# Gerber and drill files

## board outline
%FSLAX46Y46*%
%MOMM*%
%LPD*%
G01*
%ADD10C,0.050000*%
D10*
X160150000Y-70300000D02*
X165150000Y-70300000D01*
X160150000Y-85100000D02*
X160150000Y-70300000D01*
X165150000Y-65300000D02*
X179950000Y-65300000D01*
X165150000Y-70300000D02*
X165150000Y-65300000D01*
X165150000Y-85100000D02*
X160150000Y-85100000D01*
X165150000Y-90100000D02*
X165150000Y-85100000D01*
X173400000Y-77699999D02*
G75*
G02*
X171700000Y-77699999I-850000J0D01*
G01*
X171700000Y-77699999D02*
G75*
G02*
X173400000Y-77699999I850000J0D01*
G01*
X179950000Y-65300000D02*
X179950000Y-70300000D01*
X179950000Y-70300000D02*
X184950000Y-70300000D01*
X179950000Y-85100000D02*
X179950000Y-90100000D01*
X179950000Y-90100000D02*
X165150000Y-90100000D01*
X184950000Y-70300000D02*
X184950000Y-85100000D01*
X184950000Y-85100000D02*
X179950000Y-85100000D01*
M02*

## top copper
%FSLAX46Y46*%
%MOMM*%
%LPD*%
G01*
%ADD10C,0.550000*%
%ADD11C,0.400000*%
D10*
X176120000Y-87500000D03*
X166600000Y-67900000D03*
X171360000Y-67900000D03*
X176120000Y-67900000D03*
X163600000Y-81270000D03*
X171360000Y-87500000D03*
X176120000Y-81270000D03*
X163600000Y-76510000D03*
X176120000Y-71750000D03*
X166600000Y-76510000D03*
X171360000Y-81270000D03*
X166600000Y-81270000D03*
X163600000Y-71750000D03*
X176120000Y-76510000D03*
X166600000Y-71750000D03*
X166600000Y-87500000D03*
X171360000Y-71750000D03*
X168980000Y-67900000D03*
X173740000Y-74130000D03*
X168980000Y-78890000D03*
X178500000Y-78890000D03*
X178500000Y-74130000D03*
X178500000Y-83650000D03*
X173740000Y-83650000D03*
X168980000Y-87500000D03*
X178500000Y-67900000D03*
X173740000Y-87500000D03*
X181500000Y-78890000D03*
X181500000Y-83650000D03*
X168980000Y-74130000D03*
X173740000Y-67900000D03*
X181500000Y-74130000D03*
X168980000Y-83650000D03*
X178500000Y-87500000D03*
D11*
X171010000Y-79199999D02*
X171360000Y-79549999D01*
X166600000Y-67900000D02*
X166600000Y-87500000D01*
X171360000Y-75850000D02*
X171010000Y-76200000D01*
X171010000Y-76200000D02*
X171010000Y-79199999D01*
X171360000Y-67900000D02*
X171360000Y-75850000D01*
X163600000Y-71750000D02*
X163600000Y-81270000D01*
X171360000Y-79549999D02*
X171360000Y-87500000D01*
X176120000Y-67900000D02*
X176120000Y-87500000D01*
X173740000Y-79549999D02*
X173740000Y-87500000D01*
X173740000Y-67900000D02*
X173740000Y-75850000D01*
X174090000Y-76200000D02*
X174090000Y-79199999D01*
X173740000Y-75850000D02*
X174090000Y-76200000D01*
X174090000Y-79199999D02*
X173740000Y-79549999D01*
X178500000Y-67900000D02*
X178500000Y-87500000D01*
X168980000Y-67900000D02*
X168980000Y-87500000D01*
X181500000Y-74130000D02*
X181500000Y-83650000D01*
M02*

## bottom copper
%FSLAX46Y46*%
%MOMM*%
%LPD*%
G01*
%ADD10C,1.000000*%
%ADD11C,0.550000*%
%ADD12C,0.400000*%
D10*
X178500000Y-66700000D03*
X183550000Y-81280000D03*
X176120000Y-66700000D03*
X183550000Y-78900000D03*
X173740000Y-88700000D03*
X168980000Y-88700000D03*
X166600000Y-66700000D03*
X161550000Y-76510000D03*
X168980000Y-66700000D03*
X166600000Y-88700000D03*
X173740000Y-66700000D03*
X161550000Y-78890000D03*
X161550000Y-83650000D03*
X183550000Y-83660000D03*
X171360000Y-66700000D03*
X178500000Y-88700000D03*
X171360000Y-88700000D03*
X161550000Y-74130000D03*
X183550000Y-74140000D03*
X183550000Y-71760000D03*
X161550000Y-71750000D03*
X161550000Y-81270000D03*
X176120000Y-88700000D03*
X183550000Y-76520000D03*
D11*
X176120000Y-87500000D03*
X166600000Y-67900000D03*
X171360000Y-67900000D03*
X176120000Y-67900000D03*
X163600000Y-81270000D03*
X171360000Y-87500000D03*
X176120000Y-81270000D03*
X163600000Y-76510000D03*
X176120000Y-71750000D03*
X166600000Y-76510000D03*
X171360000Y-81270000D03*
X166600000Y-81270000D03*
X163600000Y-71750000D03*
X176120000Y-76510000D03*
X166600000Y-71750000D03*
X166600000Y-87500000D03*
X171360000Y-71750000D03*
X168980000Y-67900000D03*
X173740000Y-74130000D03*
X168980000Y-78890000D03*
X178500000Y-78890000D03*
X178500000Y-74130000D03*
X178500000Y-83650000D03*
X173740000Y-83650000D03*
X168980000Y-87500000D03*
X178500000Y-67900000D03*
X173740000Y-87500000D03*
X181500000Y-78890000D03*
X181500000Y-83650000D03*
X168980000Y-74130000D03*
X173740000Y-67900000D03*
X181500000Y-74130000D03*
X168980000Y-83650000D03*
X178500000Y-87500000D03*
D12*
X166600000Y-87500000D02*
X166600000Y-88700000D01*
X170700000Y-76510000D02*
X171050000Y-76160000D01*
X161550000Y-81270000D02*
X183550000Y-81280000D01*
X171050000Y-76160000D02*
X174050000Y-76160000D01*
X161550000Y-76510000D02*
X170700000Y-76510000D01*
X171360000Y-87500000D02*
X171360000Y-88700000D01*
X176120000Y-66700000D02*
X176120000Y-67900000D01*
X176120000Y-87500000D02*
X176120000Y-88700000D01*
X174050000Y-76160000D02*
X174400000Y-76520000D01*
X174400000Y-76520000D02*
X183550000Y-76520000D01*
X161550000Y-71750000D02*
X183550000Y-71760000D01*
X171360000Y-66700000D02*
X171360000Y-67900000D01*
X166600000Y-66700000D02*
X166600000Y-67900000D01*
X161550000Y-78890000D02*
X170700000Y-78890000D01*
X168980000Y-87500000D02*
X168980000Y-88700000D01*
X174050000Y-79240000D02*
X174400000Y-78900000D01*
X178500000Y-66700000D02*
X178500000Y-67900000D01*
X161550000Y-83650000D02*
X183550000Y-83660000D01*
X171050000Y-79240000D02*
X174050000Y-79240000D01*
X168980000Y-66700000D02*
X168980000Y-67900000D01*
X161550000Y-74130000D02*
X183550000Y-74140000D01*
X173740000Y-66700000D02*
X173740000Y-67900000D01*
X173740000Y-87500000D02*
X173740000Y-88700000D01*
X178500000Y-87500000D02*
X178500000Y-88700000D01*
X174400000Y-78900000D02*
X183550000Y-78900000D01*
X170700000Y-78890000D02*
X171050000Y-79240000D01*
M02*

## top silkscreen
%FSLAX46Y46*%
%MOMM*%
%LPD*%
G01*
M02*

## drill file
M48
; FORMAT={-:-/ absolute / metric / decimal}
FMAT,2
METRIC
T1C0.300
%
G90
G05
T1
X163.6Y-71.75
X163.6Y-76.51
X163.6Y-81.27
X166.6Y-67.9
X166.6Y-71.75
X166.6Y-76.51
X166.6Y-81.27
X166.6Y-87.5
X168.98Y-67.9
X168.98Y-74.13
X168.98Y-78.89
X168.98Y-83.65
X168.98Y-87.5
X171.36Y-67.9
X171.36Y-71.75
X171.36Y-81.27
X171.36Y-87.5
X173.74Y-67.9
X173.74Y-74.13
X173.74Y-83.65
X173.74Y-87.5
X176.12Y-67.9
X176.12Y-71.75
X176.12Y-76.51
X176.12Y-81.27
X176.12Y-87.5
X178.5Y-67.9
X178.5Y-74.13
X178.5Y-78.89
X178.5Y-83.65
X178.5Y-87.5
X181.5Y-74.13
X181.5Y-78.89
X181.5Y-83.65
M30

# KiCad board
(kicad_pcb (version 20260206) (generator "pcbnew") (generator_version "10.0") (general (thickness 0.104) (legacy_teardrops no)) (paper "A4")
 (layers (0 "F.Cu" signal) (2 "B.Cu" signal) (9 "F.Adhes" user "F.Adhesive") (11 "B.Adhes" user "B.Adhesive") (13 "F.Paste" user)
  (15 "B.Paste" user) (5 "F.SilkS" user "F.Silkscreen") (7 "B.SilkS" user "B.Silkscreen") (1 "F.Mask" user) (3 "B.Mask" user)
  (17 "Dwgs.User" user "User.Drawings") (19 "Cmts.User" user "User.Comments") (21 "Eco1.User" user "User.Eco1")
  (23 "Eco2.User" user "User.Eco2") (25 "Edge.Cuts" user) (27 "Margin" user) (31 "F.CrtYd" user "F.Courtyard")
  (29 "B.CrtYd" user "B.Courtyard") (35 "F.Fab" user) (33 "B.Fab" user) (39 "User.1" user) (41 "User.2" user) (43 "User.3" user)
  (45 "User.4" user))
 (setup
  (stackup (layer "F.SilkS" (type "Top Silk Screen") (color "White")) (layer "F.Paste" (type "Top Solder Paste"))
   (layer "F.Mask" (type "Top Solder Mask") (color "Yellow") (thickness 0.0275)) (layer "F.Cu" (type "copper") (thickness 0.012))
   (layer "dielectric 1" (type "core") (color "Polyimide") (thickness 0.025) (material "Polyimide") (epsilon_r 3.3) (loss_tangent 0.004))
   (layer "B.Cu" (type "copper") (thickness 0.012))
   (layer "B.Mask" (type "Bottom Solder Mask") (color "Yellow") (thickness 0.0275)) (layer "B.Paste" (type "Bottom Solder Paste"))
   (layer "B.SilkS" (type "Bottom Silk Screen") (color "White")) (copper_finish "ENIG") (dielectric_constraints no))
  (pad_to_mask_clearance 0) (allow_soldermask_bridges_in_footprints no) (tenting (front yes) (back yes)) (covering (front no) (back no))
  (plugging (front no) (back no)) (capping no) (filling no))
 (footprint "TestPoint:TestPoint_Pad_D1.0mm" (layer "B.Cu") (at 178.5 66.7 180)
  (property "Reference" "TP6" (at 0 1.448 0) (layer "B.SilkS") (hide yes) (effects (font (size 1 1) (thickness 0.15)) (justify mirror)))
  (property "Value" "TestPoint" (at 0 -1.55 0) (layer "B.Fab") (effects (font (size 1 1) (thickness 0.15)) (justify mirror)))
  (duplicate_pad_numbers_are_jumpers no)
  (pad "1" smd circle (at 0 0 180) (size 1 1) (layers "B.Cu" "B.Mask") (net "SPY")))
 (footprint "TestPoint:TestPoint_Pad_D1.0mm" (layer "B.Cu") (at 183.55 81.28 90)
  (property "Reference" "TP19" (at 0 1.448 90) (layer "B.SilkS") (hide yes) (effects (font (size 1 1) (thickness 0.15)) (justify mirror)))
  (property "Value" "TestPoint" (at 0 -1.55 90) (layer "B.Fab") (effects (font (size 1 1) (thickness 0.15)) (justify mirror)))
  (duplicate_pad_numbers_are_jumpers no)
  (pad "1" smd circle (at 0 0 90) (size 1 1) (layers "B.Cu" "B.Mask") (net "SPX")))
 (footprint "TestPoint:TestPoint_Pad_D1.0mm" (layer "B.Cu") (at 176.12 66.7 180)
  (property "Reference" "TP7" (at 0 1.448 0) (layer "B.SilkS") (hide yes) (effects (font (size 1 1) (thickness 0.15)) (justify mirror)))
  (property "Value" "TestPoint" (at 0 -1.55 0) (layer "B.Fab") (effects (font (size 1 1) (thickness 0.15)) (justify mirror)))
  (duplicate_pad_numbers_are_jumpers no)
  (pad "1" smd circle (at 0 0 180) (size 1 1) (layers "B.Cu" "B.Mask") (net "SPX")))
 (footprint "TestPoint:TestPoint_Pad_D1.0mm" (layer "B.Cu") (at 183.55 78.9 90)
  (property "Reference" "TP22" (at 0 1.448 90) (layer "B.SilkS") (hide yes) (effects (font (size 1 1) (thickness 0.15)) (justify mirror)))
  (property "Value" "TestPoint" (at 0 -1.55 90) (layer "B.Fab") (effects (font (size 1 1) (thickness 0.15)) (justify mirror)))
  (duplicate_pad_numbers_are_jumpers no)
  (pad "1" smd circle (at 0 0 90) (size 1 1) (layers "B.Cu" "B.Mask") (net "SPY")))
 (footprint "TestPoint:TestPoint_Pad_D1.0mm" (layer "B.Cu") (at 173.74 88.7)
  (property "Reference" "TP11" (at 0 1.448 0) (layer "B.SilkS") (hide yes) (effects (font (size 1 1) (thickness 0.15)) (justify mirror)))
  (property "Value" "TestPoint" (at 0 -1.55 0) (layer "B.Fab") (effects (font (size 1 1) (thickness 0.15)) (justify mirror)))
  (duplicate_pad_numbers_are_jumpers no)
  (pad "1" smd circle (at 0 0) (size 1 1) (layers "B.Cu" "B.Mask") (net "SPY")))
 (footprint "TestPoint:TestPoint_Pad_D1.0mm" (layer "B.Cu") (at 168.98 88.7)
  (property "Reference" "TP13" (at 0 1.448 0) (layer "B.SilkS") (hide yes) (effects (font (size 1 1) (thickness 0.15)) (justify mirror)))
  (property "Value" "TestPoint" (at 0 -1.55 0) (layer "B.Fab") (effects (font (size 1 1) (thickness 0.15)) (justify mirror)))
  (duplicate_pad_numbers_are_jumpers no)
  (pad "1" smd circle (at 0 0) (size 1 1) (layers "B.Cu" "B.Mask") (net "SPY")))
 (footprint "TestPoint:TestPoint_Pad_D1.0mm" (layer "B.Cu") (at 166.6 66.7 180)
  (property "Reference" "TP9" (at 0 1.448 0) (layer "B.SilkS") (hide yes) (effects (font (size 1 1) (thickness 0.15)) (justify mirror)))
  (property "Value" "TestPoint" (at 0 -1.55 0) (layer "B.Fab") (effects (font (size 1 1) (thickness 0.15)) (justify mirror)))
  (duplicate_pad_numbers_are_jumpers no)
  (pad "1" smd circle (at 0 0 180) (size 1 1) (layers "B.Cu" "B.Mask") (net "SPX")))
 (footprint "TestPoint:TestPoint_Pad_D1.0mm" (layer "B.Cu") (at 161.55 76.51 -90)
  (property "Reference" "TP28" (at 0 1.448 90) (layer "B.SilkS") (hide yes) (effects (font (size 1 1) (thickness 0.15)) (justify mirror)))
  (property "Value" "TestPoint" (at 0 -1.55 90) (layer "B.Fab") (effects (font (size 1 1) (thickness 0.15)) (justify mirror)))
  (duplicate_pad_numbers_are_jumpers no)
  (pad "1" smd circle (at 0 0 270) (size 1 1) (layers "B.Cu" "B.Mask") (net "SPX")))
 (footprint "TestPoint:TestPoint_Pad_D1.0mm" (layer "B.Cu") (at 168.98 66.7 180)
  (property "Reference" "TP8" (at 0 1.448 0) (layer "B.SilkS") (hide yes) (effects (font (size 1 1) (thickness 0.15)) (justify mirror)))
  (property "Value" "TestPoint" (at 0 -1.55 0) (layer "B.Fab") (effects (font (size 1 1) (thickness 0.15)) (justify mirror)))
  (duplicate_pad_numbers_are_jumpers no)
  (pad "1" smd circle (at 0 0 180) (size 1 1) (layers "B.Cu" "B.Mask") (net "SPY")))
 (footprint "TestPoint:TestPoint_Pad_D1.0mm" (layer "B.Cu") (at 166.6 88.7)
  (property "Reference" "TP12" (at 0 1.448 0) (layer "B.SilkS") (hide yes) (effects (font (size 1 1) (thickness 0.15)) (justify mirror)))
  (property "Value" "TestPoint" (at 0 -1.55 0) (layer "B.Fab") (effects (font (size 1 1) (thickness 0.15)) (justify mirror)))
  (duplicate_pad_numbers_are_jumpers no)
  (pad "1" smd circle (at 0 0) (size 1 1) (layers "B.Cu" "B.Mask") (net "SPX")))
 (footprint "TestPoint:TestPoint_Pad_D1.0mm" (layer "B.Cu") (at 173.74 66.7 180)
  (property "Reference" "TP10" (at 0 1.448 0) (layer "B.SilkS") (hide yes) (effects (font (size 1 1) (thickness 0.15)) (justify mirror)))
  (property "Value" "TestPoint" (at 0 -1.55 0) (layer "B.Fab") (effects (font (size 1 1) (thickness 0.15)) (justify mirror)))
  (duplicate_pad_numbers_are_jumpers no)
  (pad "1" smd circle (at 0 0 180) (size 1 1) (layers "B.Cu" "B.Mask") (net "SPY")))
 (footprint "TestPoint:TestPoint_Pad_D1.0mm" (layer "B.Cu") (at 161.55 78.89 -90)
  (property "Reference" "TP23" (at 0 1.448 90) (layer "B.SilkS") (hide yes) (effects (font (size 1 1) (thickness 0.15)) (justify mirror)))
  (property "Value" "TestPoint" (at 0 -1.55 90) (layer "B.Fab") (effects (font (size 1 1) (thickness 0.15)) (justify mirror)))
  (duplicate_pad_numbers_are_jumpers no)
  (pad "1" smd circle (at 0 0 270) (size 1 1) (layers "B.Cu" "B.Mask") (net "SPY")))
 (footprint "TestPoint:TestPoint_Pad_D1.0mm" (layer "B.Cu") (at 161.55 83.65 -90)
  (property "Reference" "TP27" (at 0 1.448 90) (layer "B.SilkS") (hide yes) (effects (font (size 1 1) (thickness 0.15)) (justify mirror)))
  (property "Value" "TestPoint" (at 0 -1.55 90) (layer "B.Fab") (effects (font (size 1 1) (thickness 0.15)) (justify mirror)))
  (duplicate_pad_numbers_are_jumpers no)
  (pad "1" smd circle (at 0 0 270) (size 1 1) (layers "B.Cu" "B.Mask") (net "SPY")))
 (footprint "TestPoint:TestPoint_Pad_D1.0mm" (layer "B.Cu") (at 183.55 83.66 90)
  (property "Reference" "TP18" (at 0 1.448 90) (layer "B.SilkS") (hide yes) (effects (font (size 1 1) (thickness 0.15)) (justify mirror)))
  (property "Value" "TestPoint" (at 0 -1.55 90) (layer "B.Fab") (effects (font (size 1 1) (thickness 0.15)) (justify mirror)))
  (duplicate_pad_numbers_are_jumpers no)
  (pad "1" smd circle (at 0 0 90) (size 1 1) (layers "B.Cu" "B.Mask") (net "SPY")))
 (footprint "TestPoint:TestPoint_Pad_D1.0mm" (layer "B.Cu") (at 171.36 66.7 180)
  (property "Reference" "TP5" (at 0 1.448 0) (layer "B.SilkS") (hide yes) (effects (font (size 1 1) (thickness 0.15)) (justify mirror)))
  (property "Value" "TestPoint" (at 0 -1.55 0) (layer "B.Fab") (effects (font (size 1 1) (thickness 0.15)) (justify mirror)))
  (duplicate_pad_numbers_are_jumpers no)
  (pad "1" smd circle (at 0 0 180) (size 1 1) (layers "B.Cu" "B.Mask") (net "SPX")))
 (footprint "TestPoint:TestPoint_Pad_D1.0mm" (layer "B.Cu") (at 178.5 88.7)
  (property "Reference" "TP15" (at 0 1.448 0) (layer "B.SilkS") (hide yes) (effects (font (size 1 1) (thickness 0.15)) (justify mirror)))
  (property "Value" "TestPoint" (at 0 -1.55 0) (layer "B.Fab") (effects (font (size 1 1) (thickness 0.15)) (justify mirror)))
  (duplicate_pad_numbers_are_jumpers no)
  (pad "1" smd circle (at 0 0) (size 1 1) (layers "B.Cu" "B.Mask") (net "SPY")))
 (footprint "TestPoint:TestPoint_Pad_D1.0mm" (layer "B.Cu") (at 171.36 88.7)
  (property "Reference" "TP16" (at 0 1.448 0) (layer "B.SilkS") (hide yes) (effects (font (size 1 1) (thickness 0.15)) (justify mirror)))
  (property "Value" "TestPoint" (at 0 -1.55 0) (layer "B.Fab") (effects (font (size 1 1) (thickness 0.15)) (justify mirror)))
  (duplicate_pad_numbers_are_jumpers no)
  (pad "1" smd circle (at 0 0) (size 1 1) (layers "B.Cu" "B.Mask") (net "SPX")))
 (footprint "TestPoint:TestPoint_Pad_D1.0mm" (layer "B.Cu") (at 161.55 74.13 -90)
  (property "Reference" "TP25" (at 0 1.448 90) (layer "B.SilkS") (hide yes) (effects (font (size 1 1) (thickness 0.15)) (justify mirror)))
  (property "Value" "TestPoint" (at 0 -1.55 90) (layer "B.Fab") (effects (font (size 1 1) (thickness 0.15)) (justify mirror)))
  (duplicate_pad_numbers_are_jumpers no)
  (pad "1" smd circle (at 0 0 270) (size 1 1) (layers "B.Cu" "B.Mask") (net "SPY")))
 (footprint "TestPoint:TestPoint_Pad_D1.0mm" (layer "B.Cu") (at 183.55 74.14 90)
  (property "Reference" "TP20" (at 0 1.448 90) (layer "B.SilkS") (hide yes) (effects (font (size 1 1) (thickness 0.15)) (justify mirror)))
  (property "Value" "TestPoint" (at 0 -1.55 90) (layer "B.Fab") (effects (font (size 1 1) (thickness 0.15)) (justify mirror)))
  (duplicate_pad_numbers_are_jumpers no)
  (pad "1" smd circle (at 0 0 90) (size 1 1) (layers "B.Cu" "B.Mask") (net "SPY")))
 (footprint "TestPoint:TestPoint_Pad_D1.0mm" (layer "B.Cu") (at 183.55 71.76 90)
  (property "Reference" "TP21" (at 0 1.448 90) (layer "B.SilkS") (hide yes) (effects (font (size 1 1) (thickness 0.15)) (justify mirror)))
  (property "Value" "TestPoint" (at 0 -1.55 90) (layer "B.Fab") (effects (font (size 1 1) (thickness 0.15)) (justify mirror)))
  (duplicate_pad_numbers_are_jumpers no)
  (pad "1" smd circle (at 0 0 90) (size 1 1) (layers "B.Cu" "B.Mask") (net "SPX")))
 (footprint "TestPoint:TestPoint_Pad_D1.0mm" (layer "B.Cu") (at 161.55 71.75 -90)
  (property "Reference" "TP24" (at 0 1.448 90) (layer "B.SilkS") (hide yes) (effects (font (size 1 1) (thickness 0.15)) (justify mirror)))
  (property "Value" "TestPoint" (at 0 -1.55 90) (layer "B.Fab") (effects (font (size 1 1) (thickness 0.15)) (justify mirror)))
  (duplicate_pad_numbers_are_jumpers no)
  (pad "1" smd circle (at 0 0 270) (size 1 1) (layers "B.Cu" "B.Mask") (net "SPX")))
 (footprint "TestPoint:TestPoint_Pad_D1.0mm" (layer "B.Cu") (at 161.55 81.27 -90)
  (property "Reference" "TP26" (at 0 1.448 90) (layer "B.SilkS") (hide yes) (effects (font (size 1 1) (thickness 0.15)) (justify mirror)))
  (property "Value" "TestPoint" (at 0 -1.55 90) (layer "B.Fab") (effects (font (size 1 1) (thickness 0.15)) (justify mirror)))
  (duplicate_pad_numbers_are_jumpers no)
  (pad "1" smd circle (at 0 0 270) (size 1 1) (layers "B.Cu" "B.Mask") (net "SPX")))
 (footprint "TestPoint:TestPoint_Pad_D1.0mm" (layer "B.Cu") (at 176.12 88.7)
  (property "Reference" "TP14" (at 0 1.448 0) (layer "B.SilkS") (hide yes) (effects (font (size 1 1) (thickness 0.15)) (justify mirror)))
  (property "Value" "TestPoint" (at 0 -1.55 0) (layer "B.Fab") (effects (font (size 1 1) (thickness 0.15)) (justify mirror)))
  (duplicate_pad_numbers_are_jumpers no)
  (pad "1" smd circle (at 0 0) (size 1 1) (layers "B.Cu" "B.Mask") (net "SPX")))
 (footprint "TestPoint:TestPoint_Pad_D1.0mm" (layer "B.Cu") (at 183.55 76.52 90)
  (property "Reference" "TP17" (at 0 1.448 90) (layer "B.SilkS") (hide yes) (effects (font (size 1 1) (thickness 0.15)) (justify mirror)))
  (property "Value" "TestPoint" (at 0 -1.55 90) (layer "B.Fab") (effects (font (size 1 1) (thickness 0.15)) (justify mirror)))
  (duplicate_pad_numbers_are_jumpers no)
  (pad "1" smd circle (at 0 0 90) (size 1 1) (layers "B.Cu" "B.Mask") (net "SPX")))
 (gr_line (start 160.15 70.3) (end 165.15 70.3) (stroke (width 0.05) (type default)) (layer "Edge.Cuts"))
 (gr_line (start 160.15 85.1) (end 160.15 70.3) (stroke (width 0.05) (type default)) (layer "Edge.Cuts"))
 (gr_line (start 165.15 65.3) (end 179.95 65.3) (stroke (width 0.05) (type default)) (layer "Edge.Cuts"))
 (gr_line (start 165.15 70.3) (end 165.15 65.3) (stroke (width 0.05) (type default)) (layer "Edge.Cuts"))
 (gr_line (start 165.15 85.1) (end 160.15 85.1) (stroke (width 0.05) (type default)) (layer "Edge.Cuts"))
 (gr_line (start 165.15 90.1) (end 165.15 85.1) (stroke (width 0.05) (type default)) (layer "Edge.Cuts"))
 (gr_circle (center 172.55 77.699999) (end 173.4 77.699999) (stroke (width 0.05) (type default)) (fill no) (layer "Edge.Cuts"))
 (gr_line (start 179.95 65.3) (end 179.95 70.3) (stroke (width 0.05) (type default)) (layer "Edge.Cuts"))
 (gr_line (start 179.95 70.3) (end 184.95 70.3) (stroke (width 0.05) (type default)) (layer "Edge.Cuts"))
 (gr_line (start 179.95 85.1) (end 179.95 90.1) (stroke (width 0.05) (type default)) (layer "Edge.Cuts"))
 (gr_line (start 179.95 90.1) (end 165.15 90.1) (stroke (width 0.05) (type default)) (layer "Edge.Cuts"))
 (gr_line (start 184.95 70.3) (end 184.95 85.1) (stroke (width 0.05) (type default)) (layer "Edge.Cuts"))
 (gr_line (start 184.95 85.1) (end 179.95 85.1) (stroke (width 0.05) (type default)) (layer "Edge.Cuts"))
 (segment (start 171.01 79.199999) (end 171.36 79.549999) (width 0.4) (layer "F.Cu") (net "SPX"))
 (segment (start 166.6 67.9) (end 166.6 87.5) (width 0.4) (layer "F.Cu") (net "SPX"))
 (segment (start 171.36 75.85) (end 171.01 76.2) (width 0.4) (layer "F.Cu") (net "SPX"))
 (segment (start 171.01 76.2) (end 171.01 79.199999) (width 0.4) (layer "F.Cu") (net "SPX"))
 (segment (start 171.36 67.9) (end 171.36 75.85) (width 0.4) (layer "F.Cu") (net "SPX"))
 (segment (start 163.6 71.75) (end 163.6 81.27) (width 0.4) (layer "F.Cu") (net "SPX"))
 (segment (start 171.36 79.549999) (end 171.36 87.5) (width 0.4) (layer "F.Cu") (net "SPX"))
 (segment (start 176.12 67.9) (end 176.12 87.5) (width 0.4) (layer "F.Cu") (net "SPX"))
 (via (at 176.12 87.5) (size 0.55) (drill 0.3) (layers "F.Cu" "B.Cu") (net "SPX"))
 (via (at 166.6 67.9) (size 0.55) (drill 0.3) (layers "F.Cu" "B.Cu") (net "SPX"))
 (via (at 171.36 67.9) (size 0.55) (drill 0.3) (layers "F.Cu" "B.Cu") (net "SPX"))
 (via (at 176.12 67.9) (size 0.55) (drill 0.3) (layers "F.Cu" "B.Cu") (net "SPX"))
 (via (at 163.6 81.27) (size 0.55) (drill 0.3) (layers "F.Cu" "B.Cu") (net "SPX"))
 (via (at 171.36 87.5) (size 0.55) (drill 0.3) (layers "F.Cu" "B.Cu") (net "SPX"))
 (via (at 176.12 81.27) (size 0.55) (drill 0.3) (layers "F.Cu" "B.Cu") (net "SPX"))
 (via (at 163.6 76.51) (size 0.55) (drill 0.3) (layers "F.Cu" "B.Cu") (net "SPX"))
 (via (at 176.12 71.75) (size 0.55) (drill 0.3) (layers "F.Cu" "B.Cu") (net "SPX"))
 (via (at 166.6 76.51) (size 0.55) (drill 0.3) (layers "F.Cu" "B.Cu") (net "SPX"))
 (via (at 171.36 81.27) (size 0.55) (drill 0.3) (layers "F.Cu" "B.Cu") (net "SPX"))
 (via (at 166.6 81.27) (size 0.55) (drill 0.3) (layers "F.Cu" "B.Cu") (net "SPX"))
 (via (at 163.6 71.75) (size 0.55) (drill 0.3) (layers "F.Cu" "B.Cu") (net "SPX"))
 (via (at 176.12 76.51) (size 0.55) (drill 0.3) (layers "F.Cu" "B.Cu") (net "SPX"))
 (via (at 166.6 71.75) (size 0.55) (drill 0.3) (layers "F.Cu" "B.Cu") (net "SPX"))
 (via (at 166.6 87.5) (size 0.55) (drill 0.3) (layers "F.Cu" "B.Cu") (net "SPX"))
 (via (at 171.36 71.75) (size 0.55) (drill 0.3) (layers "F.Cu" "B.Cu") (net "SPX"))
 (segment (start 166.6 87.5) (end 166.6 88.7) (width 0.4) (layer "B.Cu") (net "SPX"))
 (segment (start 170.7 76.51) (end 171.05 76.16) (width 0.4) (layer "B.Cu") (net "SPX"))
 (segment (start 161.55 81.27) (end 183.55 81.28) (width 0.4) (layer "B.Cu") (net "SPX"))
 (segment (start 171.05 76.16) (end 174.05 76.16) (width 0.4) (layer "B.Cu") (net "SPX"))
 (segment (start 161.55 76.51) (end 170.7 76.51) (width 0.4) (layer "B.Cu") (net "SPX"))
 (segment (start 171.36 87.5) (end 171.36 88.7) (width 0.4) (layer "B.Cu") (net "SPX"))
 (segment (start 176.12 66.7) (end 176.12 67.9) (width 0.4) (layer "B.Cu") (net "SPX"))
 (segment (start 176.12 87.5) (end 176.12 88.7) (width 0.4) (layer "B.Cu") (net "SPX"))
 (segment (start 174.05 76.16) (end 174.4 76.52) (width 0.4) (layer "B.Cu") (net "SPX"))
 (segment (start 174.4 76.52) (end 183.55 76.52) (width 0.4) (layer "B.Cu") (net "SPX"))
 (segment (start 161.55 71.75) (end 183.55 71.76) (width 0.4) (layer "B.Cu") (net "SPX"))
 (segment (start 171.36 66.7) (end 171.36 67.9) (width 0.4) (layer "B.Cu") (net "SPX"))
 (segment (start 166.6 66.7) (end 166.6 67.9) (width 0.4) (layer "B.Cu") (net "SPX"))
 (segment (start 173.74 79.549999) (end 173.74 87.5) (width 0.4) (layer "F.Cu") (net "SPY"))
 (segment (start 173.74 67.9) (end 173.74 75.85) (width 0.4) (layer "F.Cu") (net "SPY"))
 (segment (start 174.09 76.2) (end 174.09 79.199999) (width 0.4) (layer "F.Cu") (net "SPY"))
 (segment (start 173.74 75.85) (end 174.09 76.2) (width 0.4) (layer "F.Cu") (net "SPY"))
 (segment (start 174.09 79.199999) (end 173.74 79.549999) (width 0.4) (layer "F.Cu") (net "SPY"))
 (segment (start 178.5 67.9) (end 178.5 87.5) (width 0.4) (layer "F.Cu") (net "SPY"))
 (segment (start 168.98 67.9) (end 168.98 87.5) (width 0.4) (layer "F.Cu") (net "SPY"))
 (segment (start 181.5 74.13) (end 181.5 83.65) (width 0.4) (layer "F.Cu") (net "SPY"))
 (via (at 168.98 67.9) (size 0.55) (drill 0.3) (layers "F.Cu" "B.Cu") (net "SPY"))
 (via (at 173.74 74.13) (size 0.55) (drill 0.3) (layers "F.Cu" "B.Cu") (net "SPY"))
 (via (at 168.98 78.89) (size 0.55) (drill 0.3) (layers "F.Cu" "B.Cu") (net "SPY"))
 (via (at 178.5 78.89) (size 0.55) (drill 0.3) (layers "F.Cu" "B.Cu") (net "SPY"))
 (via (at 178.5 74.13) (size 0.55) (drill 0.3) (layers "F.Cu" "B.Cu") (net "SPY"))
 (via (at 178.5 83.65) (size 0.55) (drill 0.3) (layers "F.Cu" "B.Cu") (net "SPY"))
 (via (at 173.74 83.65) (size 0.55) (drill 0.3) (layers "F.Cu" "B.Cu") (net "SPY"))
 (via (at 168.98 87.5) (size 0.55) (drill 0.3) (layers "F.Cu" "B.Cu") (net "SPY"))
 (via (at 178.5 67.9) (size 0.55) (drill 0.3) (layers "F.Cu" "B.Cu") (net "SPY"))
 (via (at 173.74 87.5) (size 0.55) (drill 0.3) (layers "F.Cu" "B.Cu") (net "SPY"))
 (via (at 181.5 78.89) (size 0.55) (drill 0.3) (layers "F.Cu" "B.Cu") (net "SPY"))
 (via (at 181.5 83.65) (size 0.55) (drill 0.3) (layers "F.Cu" "B.Cu") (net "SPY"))
 (via (at 168.98 74.13) (size 0.55) (drill 0.3) (layers "F.Cu" "B.Cu") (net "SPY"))
 (via (at 173.74 67.9) (size 0.55) (drill 0.3) (layers "F.Cu" "B.Cu") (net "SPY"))
 (via (at 181.5 74.13) (size 0.55) (drill 0.3) (layers "F.Cu" "B.Cu") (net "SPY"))
 (via (at 168.98 83.65) (size 0.55) (drill 0.3) (layers "F.Cu" "B.Cu") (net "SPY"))
 (via (at 178.5 87.5) (size 0.55) (drill 0.3) (layers "F.Cu" "B.Cu") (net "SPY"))
 (segment (start 161.55 78.89) (end 170.7 78.89) (width 0.4) (layer "B.Cu") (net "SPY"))
 (segment (start 168.98 87.5) (end 168.98 88.7) (width 0.4) (layer "B.Cu") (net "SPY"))
 (segment (start 174.05 79.24) (end 174.4 78.9) (width 0.4) (layer "B.Cu") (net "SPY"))
 (segment (start 178.5 66.7) (end 178.5 67.9) (width 0.4) (layer "B.Cu") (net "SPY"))
 (segment (start 161.55 83.65) (end 183.55 83.66) (width 0.4) (layer "B.Cu") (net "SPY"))
 (segment (start 171.05 79.24) (end 174.05 79.24) (width 0.4) (layer "B.Cu") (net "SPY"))
 (segment (start 168.98 66.7) (end 168.98 67.9) (width 0.4) (layer "B.Cu") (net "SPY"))
 (segment (start 161.55 74.13) (end 183.55 74.14) (width 0.4) (layer "B.Cu") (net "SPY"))
 (segment (start 173.74 66.7) (end 173.74 67.9) (width 0.4) (layer "B.Cu") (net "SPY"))
 (segment (start 173.74 87.5) (end 173.74 88.7) (width 0.4) (layer "B.Cu") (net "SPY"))
 (segment (start 178.5 87.5) (end 178.5 88.7) (width 0.4) (layer "B.Cu") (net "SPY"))
 (segment (start 174.4 78.9) (end 183.55 78.9) (width 0.4) (layer "B.Cu") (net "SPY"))
 (segment (start 170.7 78.89) (end 171.05 79.24) (width 0.4) (layer "B.Cu") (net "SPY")))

